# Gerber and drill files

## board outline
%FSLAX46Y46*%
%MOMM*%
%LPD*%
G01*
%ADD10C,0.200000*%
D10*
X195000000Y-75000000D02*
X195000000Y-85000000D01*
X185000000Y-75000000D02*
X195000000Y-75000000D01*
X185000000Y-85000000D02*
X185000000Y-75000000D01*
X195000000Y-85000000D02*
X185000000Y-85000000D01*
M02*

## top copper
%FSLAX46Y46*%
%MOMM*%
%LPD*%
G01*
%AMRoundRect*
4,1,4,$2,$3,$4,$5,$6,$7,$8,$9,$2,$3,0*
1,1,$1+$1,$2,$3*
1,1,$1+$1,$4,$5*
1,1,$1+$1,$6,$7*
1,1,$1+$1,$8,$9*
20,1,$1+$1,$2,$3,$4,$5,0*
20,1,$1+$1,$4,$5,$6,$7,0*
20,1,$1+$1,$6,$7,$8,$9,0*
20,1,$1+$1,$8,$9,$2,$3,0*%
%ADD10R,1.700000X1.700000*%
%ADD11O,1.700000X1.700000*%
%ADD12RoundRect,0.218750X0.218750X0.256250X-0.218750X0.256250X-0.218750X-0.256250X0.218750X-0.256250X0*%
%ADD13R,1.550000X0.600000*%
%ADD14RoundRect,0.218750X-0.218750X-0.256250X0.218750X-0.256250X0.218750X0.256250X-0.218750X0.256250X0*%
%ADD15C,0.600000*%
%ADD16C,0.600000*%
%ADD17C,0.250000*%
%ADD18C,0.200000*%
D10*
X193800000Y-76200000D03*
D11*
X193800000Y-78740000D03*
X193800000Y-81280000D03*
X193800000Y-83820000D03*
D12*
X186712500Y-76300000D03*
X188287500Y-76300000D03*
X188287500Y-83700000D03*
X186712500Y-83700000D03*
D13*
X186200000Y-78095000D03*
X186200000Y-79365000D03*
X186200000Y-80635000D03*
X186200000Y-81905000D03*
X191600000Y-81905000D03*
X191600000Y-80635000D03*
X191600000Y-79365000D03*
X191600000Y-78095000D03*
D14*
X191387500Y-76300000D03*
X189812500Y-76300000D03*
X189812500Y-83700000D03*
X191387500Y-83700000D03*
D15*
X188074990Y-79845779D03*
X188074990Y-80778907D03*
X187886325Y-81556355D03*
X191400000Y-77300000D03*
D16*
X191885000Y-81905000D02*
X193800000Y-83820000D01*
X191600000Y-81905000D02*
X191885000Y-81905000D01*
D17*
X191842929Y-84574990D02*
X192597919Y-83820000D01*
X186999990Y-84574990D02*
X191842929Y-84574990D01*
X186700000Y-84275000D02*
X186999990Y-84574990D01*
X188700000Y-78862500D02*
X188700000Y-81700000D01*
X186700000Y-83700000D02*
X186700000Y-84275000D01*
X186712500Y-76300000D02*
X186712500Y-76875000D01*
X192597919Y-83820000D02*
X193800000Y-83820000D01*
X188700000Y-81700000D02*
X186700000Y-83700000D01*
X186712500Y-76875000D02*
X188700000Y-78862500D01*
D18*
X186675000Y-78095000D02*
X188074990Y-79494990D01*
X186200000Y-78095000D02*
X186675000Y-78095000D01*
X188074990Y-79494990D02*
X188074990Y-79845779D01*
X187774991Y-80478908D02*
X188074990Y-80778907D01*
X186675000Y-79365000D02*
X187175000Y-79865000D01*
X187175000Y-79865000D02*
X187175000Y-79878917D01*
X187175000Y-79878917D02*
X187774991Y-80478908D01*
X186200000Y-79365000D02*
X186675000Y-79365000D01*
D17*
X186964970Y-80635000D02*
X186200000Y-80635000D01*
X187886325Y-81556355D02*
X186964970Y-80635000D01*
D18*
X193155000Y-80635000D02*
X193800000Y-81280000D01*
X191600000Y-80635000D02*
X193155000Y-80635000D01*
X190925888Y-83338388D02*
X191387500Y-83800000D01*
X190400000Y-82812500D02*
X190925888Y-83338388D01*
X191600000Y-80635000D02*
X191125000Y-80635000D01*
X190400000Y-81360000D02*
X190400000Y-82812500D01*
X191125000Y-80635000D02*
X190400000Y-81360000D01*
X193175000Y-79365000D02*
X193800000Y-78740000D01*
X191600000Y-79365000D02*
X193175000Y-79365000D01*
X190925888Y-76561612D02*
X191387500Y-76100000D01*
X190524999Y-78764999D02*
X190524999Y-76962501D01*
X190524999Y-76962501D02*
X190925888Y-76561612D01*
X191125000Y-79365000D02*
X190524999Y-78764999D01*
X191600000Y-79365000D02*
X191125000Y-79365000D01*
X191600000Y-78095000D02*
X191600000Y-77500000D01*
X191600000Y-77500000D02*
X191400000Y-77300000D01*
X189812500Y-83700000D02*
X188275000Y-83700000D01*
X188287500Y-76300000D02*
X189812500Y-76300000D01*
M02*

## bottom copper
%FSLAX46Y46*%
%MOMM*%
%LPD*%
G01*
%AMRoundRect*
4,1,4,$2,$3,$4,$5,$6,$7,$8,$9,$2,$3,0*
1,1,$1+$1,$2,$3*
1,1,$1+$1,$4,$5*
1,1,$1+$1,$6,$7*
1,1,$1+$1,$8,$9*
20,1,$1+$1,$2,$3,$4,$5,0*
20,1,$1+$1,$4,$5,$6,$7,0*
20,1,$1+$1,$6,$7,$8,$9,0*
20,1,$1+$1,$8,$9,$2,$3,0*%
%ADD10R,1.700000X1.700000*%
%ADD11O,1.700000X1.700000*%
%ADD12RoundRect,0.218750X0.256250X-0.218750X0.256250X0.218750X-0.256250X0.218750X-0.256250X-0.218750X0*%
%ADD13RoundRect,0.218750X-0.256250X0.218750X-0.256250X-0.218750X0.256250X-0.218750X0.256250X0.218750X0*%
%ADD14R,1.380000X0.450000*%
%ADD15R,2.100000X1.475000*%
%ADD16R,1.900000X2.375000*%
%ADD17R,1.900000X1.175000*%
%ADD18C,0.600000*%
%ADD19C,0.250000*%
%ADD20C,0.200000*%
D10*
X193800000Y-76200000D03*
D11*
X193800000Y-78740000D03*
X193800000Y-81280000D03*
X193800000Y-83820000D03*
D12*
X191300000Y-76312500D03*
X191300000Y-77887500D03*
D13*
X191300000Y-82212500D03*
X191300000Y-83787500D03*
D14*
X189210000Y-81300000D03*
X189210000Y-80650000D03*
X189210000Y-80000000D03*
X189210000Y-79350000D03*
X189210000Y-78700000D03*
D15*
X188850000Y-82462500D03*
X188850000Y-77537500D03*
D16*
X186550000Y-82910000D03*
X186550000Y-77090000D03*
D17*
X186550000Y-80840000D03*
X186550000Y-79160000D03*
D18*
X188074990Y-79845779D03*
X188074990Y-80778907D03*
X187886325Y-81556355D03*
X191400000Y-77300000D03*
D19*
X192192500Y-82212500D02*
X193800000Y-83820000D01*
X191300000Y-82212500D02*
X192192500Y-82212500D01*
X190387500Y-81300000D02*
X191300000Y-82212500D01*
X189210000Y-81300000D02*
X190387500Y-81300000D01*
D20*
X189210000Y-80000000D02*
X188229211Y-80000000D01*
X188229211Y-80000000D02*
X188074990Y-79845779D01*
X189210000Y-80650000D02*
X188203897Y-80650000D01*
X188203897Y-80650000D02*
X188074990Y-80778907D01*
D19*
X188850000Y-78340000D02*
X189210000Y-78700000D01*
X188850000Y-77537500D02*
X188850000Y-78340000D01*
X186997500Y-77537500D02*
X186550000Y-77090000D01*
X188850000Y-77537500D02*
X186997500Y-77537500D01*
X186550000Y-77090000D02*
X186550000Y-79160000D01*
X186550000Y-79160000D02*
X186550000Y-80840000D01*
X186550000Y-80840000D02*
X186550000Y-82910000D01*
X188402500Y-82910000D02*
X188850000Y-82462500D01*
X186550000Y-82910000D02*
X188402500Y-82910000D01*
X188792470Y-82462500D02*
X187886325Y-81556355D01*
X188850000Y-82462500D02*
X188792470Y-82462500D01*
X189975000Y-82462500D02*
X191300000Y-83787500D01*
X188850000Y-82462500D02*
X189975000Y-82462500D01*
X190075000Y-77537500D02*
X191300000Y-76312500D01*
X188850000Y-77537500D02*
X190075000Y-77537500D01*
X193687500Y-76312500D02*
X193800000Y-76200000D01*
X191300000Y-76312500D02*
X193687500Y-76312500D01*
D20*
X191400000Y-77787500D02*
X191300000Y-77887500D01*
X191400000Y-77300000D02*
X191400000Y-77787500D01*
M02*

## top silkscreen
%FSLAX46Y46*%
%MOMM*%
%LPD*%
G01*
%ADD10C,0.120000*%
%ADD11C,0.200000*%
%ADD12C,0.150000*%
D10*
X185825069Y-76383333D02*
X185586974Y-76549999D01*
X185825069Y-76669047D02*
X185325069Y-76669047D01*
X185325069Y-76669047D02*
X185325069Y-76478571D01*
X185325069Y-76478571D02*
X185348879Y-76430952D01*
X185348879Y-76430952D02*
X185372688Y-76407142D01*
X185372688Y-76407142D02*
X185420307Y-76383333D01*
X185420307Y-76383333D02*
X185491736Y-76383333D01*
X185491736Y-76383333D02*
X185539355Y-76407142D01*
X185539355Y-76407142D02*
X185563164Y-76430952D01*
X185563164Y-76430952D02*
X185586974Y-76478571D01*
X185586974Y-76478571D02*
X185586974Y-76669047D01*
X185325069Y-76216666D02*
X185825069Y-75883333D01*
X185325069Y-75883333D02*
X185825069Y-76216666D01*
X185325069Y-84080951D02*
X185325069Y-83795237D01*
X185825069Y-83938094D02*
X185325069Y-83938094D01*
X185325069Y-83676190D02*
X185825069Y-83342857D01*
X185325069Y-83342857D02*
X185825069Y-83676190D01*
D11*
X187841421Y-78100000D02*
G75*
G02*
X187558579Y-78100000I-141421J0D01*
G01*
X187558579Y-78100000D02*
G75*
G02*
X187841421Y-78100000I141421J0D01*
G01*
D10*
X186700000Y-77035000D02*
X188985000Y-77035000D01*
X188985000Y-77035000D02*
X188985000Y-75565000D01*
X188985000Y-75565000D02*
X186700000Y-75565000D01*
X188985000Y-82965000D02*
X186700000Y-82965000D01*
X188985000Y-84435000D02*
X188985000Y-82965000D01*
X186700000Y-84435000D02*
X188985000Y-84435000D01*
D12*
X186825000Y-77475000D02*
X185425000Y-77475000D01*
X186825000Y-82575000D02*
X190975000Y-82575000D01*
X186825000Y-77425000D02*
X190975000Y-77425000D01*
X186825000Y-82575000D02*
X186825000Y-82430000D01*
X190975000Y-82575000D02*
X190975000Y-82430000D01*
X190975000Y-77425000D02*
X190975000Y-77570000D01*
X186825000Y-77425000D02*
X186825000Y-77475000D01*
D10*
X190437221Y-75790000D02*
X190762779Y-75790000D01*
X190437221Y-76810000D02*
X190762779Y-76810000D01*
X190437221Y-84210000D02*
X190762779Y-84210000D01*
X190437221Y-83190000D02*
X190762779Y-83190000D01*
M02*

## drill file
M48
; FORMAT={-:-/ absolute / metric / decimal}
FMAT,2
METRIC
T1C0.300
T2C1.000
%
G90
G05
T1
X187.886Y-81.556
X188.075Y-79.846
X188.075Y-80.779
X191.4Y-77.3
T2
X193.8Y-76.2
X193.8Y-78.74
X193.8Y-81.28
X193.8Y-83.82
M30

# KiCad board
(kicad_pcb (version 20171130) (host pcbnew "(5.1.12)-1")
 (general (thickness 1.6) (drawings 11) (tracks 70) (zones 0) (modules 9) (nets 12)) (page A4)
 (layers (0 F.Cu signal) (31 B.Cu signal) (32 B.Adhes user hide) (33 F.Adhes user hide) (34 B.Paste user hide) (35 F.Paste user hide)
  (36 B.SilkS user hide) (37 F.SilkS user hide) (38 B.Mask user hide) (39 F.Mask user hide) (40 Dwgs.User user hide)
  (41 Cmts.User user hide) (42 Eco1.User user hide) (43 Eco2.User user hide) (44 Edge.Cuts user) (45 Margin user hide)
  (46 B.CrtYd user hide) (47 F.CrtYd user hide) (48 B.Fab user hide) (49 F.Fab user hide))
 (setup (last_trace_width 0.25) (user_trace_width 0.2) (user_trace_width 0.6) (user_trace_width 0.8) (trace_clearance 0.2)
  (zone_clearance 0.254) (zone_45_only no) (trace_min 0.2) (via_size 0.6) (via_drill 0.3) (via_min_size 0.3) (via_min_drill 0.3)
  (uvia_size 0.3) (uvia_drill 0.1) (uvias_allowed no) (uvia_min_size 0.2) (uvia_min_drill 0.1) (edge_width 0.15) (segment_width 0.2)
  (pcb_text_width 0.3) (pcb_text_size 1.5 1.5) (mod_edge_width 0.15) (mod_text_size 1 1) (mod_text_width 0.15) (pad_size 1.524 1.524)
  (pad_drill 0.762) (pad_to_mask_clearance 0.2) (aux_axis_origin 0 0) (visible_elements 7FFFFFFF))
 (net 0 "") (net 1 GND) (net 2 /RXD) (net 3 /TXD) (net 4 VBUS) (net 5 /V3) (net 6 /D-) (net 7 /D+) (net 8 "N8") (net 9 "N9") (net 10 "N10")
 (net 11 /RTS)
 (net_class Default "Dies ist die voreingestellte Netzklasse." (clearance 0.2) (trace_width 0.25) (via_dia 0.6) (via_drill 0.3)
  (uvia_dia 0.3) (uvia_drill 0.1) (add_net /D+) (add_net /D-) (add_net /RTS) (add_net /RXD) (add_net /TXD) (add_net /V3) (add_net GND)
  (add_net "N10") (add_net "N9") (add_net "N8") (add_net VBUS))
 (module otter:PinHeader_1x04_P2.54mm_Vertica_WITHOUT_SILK (layer F.Cu) (at 193.8 76.2)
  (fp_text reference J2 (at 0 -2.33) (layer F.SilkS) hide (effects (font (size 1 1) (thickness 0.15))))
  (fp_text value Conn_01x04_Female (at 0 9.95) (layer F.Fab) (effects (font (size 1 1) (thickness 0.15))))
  (pad 1 thru_hole rect (at 0 0) (size 1.7 1.7) (drill 1) (layers *.Cu *.Mask) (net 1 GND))
  (pad 2 thru_hole oval (at 0 2.54) (size 1.7 1.7) (drill 1) (layers *.Cu *.Mask) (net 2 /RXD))
  (pad 3 thru_hole oval (at 0 5.08) (size 1.7 1.7) (drill 1) (layers *.Cu *.Mask) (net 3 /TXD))
  (pad 4 thru_hole oval (at 0 7.62) (size 1.7 1.7) (drill 1) (layers *.Cu *.Mask) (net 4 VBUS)))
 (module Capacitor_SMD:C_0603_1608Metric (layer B.Cu) (at 191.3 77.1 90)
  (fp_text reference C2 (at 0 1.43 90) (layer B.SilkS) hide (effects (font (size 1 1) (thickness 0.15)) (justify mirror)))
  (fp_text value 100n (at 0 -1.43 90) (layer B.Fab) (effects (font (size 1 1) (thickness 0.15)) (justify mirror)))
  (pad 2 smd roundrect (at 0.7875 0 90) (size 0.875 0.95) (layers B.Cu B.Paste B.Mask) (roundrect_rratio 0.25) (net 1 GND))
  (pad 1 smd roundrect (at -0.7875 0 90) (size 0.875 0.95) (layers B.Cu B.Paste B.Mask) (roundrect_rratio 0.25) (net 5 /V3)))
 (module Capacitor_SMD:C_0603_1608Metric (layer B.Cu) (at 191.3 83 270)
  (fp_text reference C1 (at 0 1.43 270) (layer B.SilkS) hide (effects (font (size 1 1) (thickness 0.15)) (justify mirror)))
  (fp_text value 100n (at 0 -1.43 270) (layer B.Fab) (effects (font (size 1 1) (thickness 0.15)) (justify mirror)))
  (pad 1 smd roundrect (at -0.7875 0 270) (size 0.875 0.95) (layers B.Cu B.Paste B.Mask) (roundrect_rratio 0.25) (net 4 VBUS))
  (pad 2 smd roundrect (at 0.7875 0 270) (size 0.875 0.95) (layers B.Cu B.Paste B.Mask) (roundrect_rratio 0.25) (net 1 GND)))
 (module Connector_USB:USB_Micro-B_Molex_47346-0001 (layer B.Cu) (at 187.75 80 90)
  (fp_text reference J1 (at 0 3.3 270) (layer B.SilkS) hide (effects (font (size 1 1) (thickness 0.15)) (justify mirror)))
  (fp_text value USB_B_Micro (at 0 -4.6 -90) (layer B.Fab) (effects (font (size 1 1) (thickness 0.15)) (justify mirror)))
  (pad 1 smd rect (at -1.3 1.46 90) (size 0.45 1.38) (layers B.Cu B.Paste B.Mask) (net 4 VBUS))
  (pad 2 smd rect (at -0.65 1.46 90) (size 0.45 1.38) (layers B.Cu B.Paste B.Mask) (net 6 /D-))
  (pad 3 smd rect (at 0 1.46 90) (size 0.45 1.38) (layers B.Cu B.Paste B.Mask) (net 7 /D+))
  (pad 4 smd rect (at 0.65 1.46 90) (size 0.45 1.38) (layers B.Cu B.Paste B.Mask) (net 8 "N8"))
  (pad 5 smd rect (at 1.3 1.46 90) (size 0.45 1.38) (layers B.Cu B.Paste B.Mask) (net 1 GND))
  (pad 6 smd rect (at -2.4625 1.1 90) (size 1.475 2.1) (layers B.Cu B.Paste B.Mask) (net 1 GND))
  (pad 6 smd rect (at 2.4625 1.1 90) (size 1.475 2.1) (layers B.Cu B.Paste B.Mask) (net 1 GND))
  (pad 6 smd rect (at -2.91 -1.2 90) (size 2.375 1.9) (layers B.Cu B.Paste B.Mask) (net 1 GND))
  (pad 6 smd rect (at 2.91 -1.2 90) (size 2.375 1.9) (layers B.Cu B.Paste B.Mask) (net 1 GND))
  (pad 6 smd rect (at -0.84 -1.2 90) (size 1.175 1.9) (layers B.Cu B.Paste B.Mask) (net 1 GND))
  (pad 6 smd rect (at 0.84 -1.2 90) (size 1.175 1.9) (layers B.Cu B.Paste B.Mask) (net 1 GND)))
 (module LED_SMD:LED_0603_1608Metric (layer F.Cu) (at 187.5 76.3 180)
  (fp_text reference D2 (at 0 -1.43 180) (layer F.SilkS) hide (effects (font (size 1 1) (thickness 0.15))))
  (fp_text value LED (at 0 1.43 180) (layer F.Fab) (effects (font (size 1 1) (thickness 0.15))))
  (fp_line (start 0.8 -0.735) (end -1.485 -0.735) (layer F.SilkS) (width 0.12))
  (fp_line (start -1.485 -0.735) (end -1.485 0.735) (layer F.SilkS) (width 0.12))
  (fp_line (start -1.485 0.735) (end 0.8 0.735) (layer F.SilkS) (width 0.12))
  (pad 2 smd roundrect (at 0.7875 0 180) (size 0.875 0.95) (layers F.Cu F.Paste F.Mask) (roundrect_rratio 0.25) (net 4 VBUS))
  (pad 1 smd roundrect (at -0.7875 0 180) (size 0.875 0.95) (layers F.Cu F.Paste F.Mask) (roundrect_rratio 0.25) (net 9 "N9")))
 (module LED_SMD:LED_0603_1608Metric (layer F.Cu) (at 187.5 83.7 180)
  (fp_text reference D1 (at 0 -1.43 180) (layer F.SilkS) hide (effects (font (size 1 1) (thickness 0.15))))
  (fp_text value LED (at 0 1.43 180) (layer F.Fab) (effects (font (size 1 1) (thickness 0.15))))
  (fp_line (start -1.485 0.735) (end 0.8 0.735) (layer F.SilkS) (width 0.12))
  (fp_line (start -1.485 -0.735) (end -1.485 0.735) (layer F.SilkS) (width 0.12))
  (fp_line (start 0.8 -0.735) (end -1.485 -0.735) (layer F.SilkS) (width 0.12))
  (pad 1 smd roundrect (at -0.7875 0 180) (size 0.875 0.95) (layers F.Cu F.Paste F.Mask) (roundrect_rratio 0.25) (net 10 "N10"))
  (pad 2 smd roundrect (at 0.7875 0 180) (size 0.875 0.95) (layers F.Cu F.Paste F.Mask) (roundrect_rratio 0.25) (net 4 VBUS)))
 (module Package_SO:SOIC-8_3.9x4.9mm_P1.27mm (layer F.Cu) (at 188.9 80)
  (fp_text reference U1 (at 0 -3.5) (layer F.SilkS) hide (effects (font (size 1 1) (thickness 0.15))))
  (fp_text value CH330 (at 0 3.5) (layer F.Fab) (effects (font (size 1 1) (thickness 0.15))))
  (fp_line (start -2.075 -2.525) (end -3.475 -2.525) (layer F.SilkS) (width 0.15))
  (fp_line (start -2.075 2.575) (end 2.075 2.575) (layer F.SilkS) (width 0.15))
  (fp_line (start -2.075 -2.575) (end 2.075 -2.575) (layer F.SilkS) (width 0.15))
  (fp_line (start -2.075 2.575) (end -2.075 2.43) (layer F.SilkS) (width 0.15))
  (fp_line (start 2.075 2.575) (end 2.075 2.43) (layer F.SilkS) (width 0.15))
  (fp_line (start 2.075 -2.575) (end 2.075 -2.43) (layer F.SilkS) (width 0.15))
  (fp_line (start -2.075 -2.575) (end -2.075 -2.525) (layer F.SilkS) (width 0.15))
  (pad 1 smd rect (at -2.7 -1.905) (size 1.55 0.6) (layers F.Cu F.Paste F.Mask) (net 7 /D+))
  (pad 2 smd rect (at -2.7 -0.635) (size 1.55 0.6) (layers F.Cu F.Paste F.Mask) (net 6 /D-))
  (pad 3 smd rect (at -2.7 0.635) (size 1.55 0.6) (layers F.Cu F.Paste F.Mask) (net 1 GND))
  (pad 4 smd rect (at -2.7 1.905) (size 1.55 0.6) (layers F.Cu F.Paste F.Mask) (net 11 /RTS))
  (pad 5 smd rect (at 2.7 1.905) (size 1.55 0.6) (layers F.Cu F.Paste F.Mask) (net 4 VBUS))
  (pad 6 smd rect (at 2.7 0.635) (size 1.55 0.6) (layers F.Cu F.Paste F.Mask) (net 3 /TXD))
  (pad 7 smd rect (at 2.7 -0.635) (size 1.55 0.6) (layers F.Cu F.Paste F.Mask) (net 2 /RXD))
  (pad 8 smd rect (at 2.7 -1.905) (size 1.55 0.6) (layers F.Cu F.Paste F.Mask) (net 5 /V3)))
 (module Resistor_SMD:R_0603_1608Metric (layer F.Cu) (at 190.6 76.3)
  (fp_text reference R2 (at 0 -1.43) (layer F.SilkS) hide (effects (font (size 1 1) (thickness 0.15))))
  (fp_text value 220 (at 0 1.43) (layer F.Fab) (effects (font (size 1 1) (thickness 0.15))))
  (fp_line (start -0.162779 -0.51) (end 0.162779 -0.51) (layer F.SilkS) (width 0.12))
  (fp_line (start -0.162779 0.51) (end 0.162779 0.51) (layer F.SilkS) (width 0.12))
  (pad 2 smd roundrect (at 0.7875 0) (size 0.875 0.95) (layers F.Cu F.Paste F.Mask) (roundrect_rratio 0.25) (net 2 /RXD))
  (pad 1 smd roundrect (at -0.7875 0) (size 0.875 0.95) (layers F.Cu F.Paste F.Mask) (roundrect_rratio 0.25) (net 9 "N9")))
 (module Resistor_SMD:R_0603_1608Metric (layer F.Cu) (at 190.6 83.7)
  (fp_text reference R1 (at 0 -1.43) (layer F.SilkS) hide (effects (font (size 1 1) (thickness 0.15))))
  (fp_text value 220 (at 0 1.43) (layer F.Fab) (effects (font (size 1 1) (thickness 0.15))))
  (fp_line (start -0.162779 0.51) (end 0.162779 0.51) (layer F.SilkS) (width 0.12))
  (fp_line (start -0.162779 -0.51) (end 0.162779 -0.51) (layer F.SilkS) (width 0.12))
  (pad 1 smd roundrect (at -0.7875 0) (size 0.875 0.95) (layers F.Cu F.Paste F.Mask) (roundrect_rratio 0.25) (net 10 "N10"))
  (pad 2 smd roundrect (at 0.7875 0) (size 0.875 0.95) (layers F.Cu F.Paste F.Mask) (roundrect_rratio 0.25) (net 3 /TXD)))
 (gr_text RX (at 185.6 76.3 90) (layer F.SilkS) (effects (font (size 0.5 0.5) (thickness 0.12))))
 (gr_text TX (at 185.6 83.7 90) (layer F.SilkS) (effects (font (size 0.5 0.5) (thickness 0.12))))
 (gr_circle (center 187.7 78.1) (end 187.8 78.2) (layer F.SilkS) (width 0.2))
 (gr_line (start 195 75) (end 195 85) (layer Edge.Cuts) (width 0.2))
 (gr_line (start 185 75) (end 195 75) (layer Edge.Cuts) (width 0.2))
 (gr_line (start 185 85) (end 185 75) (layer Edge.Cuts) (width 0.2))
 (gr_line (start 195 85) (end 185 85) (layer Edge.Cuts) (width 0.2))
 (segment (start 191.885 81.905) (end 193.8 83.82) (width 0.6) (layer F.Cu) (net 4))
 (segment (start 191.6 81.905) (end 191.885 81.905) (width 0.6) (layer F.Cu) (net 4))
 (segment (start 191.842929 84.57499) (end 192.597919 83.82) (width 0.25) (layer F.Cu) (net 4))
 (segment (start 186.99999 84.57499) (end 191.842929 84.57499) (width 0.25) (layer F.Cu) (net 4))
 (segment (start 186.7 84.275) (end 186.99999 84.57499) (width 0.25) (layer F.Cu) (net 4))
 (segment (start 188.7 78.8625) (end 188.7 81.7) (width 0.25) (layer F.Cu) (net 4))
 (segment (start 186.7 83.7) (end 186.7 84.275) (width 0.25) (layer F.Cu) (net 4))
 (segment (start 186.7125 76.3) (end 186.7125 76.875) (width 0.25) (layer F.Cu) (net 4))
 (segment (start 192.597919 83.82) (end 193.8 83.82) (width 0.25) (layer F.Cu) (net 4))
 (segment (start 188.7 81.7) (end 186.7 83.7) (width 0.25) (layer F.Cu) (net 4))
 (segment (start 186.7125 76.875) (end 188.7 78.8625) (width 0.25) (layer F.Cu) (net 4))
 (segment (start 192.1925 82.2125) (end 193.8 83.82) (width 0.25) (layer B.Cu) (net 4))
 (segment (start 191.3 82.2125) (end 192.1925 82.2125) (width 0.25) (layer B.Cu) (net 4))
 (segment (start 190.3875 81.3) (end 191.3 82.2125) (width 0.25) (layer B.Cu) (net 4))
 (segment (start 189.21 81.3) (end 190.3875 81.3) (width 0.25) (layer B.Cu) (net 4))
 (segment (start 186.675 78.095) (end 188.07499 79.49499) (width 0.2) (layer F.Cu) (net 7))
 (segment (start 189.21 80) (end 188.229211 80) (width 0.2) (layer B.Cu) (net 7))
 (segment (start 188.229211 80) (end 188.07499 79.845779) (width 0.2) (layer B.Cu) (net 7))
 (segment (start 186.2 78.095) (end 186.675 78.095) (width 0.2) (layer F.Cu) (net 7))
 (segment (start 188.07499 79.49499) (end 188.07499 79.845779) (width 0.2) (layer F.Cu) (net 7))
 (segment (start 187.774991 80.478908) (end 188.07499 80.778907) (width 0.2) (layer F.Cu) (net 6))
 (segment (start 189.21 80.65) (end 188.203897 80.65) (width 0.2) (layer B.Cu) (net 6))
 (segment (start 186.675 79.365) (end 187.175 79.865) (width 0.2) (layer F.Cu) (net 6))
 (segment (start 187.175 79.865) (end 187.175 79.878917) (width 0.2) (layer F.Cu) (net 6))
 (segment (start 187.175 79.878917) (end 187.774991 80.478908) (width 0.2) (layer F.Cu) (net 6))
 (segment (start 186.2 79.365) (end 186.675 79.365) (width 0.2) (layer F.Cu) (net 6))
 (segment (start 188.203897 80.65) (end 188.07499 80.778907) (width 0.2) (layer B.Cu) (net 6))
 (segment (start 188.85 78.34) (end 189.21 78.7) (width 0.25) (layer B.Cu) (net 1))
 (segment (start 188.85 77.5375) (end 188.85 78.34) (width 0.25) (layer B.Cu) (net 1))
 (segment (start 186.9975 77.5375) (end 186.55 77.09) (width 0.25) (layer B.Cu) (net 1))
 (segment (start 188.85 77.5375) (end 186.9975 77.5375) (width 0.25) (layer B.Cu) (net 1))
 (segment (start 186.55 77.09) (end 186.55 79.16) (width 0.25) (layer B.Cu) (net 1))
 (segment (start 186.55 79.16) (end 186.55 80.84) (width 0.25) (layer B.Cu) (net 1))
 (segment (start 186.55 80.84) (end 186.55 82.91) (width 0.25) (layer B.Cu) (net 1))
 (segment (start 188.4025 82.91) (end 188.85 82.4625) (width 0.25) (layer B.Cu) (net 1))
 (segment (start 186.55 82.91) (end 188.4025 82.91) (width 0.25) (layer B.Cu) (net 1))
 (segment (start 188.79247 82.4625) (end 187.886325 81.556355) (width 0.25) (layer B.Cu) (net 1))
 (segment (start 188.85 82.4625) (end 188.79247 82.4625) (width 0.25) (layer B.Cu) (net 1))
 (segment (start 189.975 82.4625) (end 191.3 83.7875) (width 0.25) (layer B.Cu) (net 1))
 (segment (start 188.85 82.4625) (end 189.975 82.4625) (width 0.25) (layer B.Cu) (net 1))
 (segment (start 190.075 77.5375) (end 191.3 76.3125) (width 0.25) (layer B.Cu) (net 1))
 (segment (start 188.85 77.5375) (end 190.075 77.5375) (width 0.25) (layer B.Cu) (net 1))
 (segment (start 193.6875 76.3125) (end 193.8 76.2) (width 0.25) (layer B.Cu) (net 1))
 (segment (start 191.3 76.3125) (end 193.6875 76.3125) (width 0.25) (layer B.Cu) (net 1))
 (segment (start 186.96497 80.635) (end 186.2 80.635) (width 0.25) (layer F.Cu) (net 1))
 (segment (start 187.886325 81.556355) (end 186.96497 80.635) (width 0.25) (layer F.Cu) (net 1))
 (segment (start 193.155 80.635) (end 193.8 81.28) (width 0.2) (layer F.Cu) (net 3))
 (segment (start 191.6 80.635) (end 193.155 80.635) (width 0.2) (layer F.Cu) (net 3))
 (segment (start 190.925888 83.338388) (end 191.3875 83.8) (width 0.2) (layer F.Cu) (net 3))
 (segment (start 190.4 82.8125) (end 190.925888 83.338388) (width 0.2) (layer F.Cu) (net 3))
 (segment (start 191.6 80.635) (end 191.125 80.635) (width 0.2) (layer F.Cu) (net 3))
 (segment (start 190.4 81.36) (end 190.4 82.8125) (width 0.2) (layer F.Cu) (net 3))
 (segment (start 191.125 80.635) (end 190.4 81.36) (width 0.2) (layer F.Cu) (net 3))
 (segment (start 193.175 79.365) (end 193.8 78.74) (width 0.2) (layer F.Cu) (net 2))
 (segment (start 191.6 79.365) (end 193.175 79.365) (width 0.2) (layer F.Cu) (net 2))
 (segment (start 190.925888 76.561612) (end 191.3875 76.1) (width 0.2) (layer F.Cu) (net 2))
 (segment (start 190.524999 78.764999) (end 190.524999 76.962501) (width 0.2) (layer F.Cu) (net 2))
 (segment (start 190.524999 76.962501) (end 190.925888 76.561612) (width 0.2) (layer F.Cu) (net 2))
 (segment (start 191.125 79.365) (end 190.524999 78.764999) (width 0.2) (layer F.Cu) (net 2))
 (segment (start 191.6 79.365) (end 191.125 79.365) (width 0.2) (layer F.Cu) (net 2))
 (segment (start 191.6 78.095) (end 191.6 77.5) (width 0.2) (layer F.Cu) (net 5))
 (segment (start 191.6 77.5) (end 191.4 77.3) (width 0.2) (layer F.Cu) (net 5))
 (segment (start 191.4 77.7875) (end 191.3 77.8875) (width 0.2) (layer B.Cu) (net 5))
 (segment (start 191.4 77.3) (end 191.4 77.7875) (width 0.2) (layer B.Cu) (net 5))
 (segment (start 189.8125 83.7) (end 188.275 83.7) (width 0.2) (layer F.Cu) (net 10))
 (segment (start 188.2875 76.3) (end 189.8125 76.3) (width 0.2) (layer F.Cu) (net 9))
 (via (at 188.07499 79.845779) (size 0.6) (drill 0.3) (layers F.Cu B.Cu) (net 7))
 (via (at 188.07499 80.778907) (size 0.6) (drill 0.3) (layers F.Cu B.Cu) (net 6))
 (via (at 187.886325 81.556355) (size 0.6) (drill 0.3) (layers F.Cu B.Cu) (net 1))
 (via (at 191.4 77.3) (size 0.6) (drill 0.3) (layers F.Cu B.Cu) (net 5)))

